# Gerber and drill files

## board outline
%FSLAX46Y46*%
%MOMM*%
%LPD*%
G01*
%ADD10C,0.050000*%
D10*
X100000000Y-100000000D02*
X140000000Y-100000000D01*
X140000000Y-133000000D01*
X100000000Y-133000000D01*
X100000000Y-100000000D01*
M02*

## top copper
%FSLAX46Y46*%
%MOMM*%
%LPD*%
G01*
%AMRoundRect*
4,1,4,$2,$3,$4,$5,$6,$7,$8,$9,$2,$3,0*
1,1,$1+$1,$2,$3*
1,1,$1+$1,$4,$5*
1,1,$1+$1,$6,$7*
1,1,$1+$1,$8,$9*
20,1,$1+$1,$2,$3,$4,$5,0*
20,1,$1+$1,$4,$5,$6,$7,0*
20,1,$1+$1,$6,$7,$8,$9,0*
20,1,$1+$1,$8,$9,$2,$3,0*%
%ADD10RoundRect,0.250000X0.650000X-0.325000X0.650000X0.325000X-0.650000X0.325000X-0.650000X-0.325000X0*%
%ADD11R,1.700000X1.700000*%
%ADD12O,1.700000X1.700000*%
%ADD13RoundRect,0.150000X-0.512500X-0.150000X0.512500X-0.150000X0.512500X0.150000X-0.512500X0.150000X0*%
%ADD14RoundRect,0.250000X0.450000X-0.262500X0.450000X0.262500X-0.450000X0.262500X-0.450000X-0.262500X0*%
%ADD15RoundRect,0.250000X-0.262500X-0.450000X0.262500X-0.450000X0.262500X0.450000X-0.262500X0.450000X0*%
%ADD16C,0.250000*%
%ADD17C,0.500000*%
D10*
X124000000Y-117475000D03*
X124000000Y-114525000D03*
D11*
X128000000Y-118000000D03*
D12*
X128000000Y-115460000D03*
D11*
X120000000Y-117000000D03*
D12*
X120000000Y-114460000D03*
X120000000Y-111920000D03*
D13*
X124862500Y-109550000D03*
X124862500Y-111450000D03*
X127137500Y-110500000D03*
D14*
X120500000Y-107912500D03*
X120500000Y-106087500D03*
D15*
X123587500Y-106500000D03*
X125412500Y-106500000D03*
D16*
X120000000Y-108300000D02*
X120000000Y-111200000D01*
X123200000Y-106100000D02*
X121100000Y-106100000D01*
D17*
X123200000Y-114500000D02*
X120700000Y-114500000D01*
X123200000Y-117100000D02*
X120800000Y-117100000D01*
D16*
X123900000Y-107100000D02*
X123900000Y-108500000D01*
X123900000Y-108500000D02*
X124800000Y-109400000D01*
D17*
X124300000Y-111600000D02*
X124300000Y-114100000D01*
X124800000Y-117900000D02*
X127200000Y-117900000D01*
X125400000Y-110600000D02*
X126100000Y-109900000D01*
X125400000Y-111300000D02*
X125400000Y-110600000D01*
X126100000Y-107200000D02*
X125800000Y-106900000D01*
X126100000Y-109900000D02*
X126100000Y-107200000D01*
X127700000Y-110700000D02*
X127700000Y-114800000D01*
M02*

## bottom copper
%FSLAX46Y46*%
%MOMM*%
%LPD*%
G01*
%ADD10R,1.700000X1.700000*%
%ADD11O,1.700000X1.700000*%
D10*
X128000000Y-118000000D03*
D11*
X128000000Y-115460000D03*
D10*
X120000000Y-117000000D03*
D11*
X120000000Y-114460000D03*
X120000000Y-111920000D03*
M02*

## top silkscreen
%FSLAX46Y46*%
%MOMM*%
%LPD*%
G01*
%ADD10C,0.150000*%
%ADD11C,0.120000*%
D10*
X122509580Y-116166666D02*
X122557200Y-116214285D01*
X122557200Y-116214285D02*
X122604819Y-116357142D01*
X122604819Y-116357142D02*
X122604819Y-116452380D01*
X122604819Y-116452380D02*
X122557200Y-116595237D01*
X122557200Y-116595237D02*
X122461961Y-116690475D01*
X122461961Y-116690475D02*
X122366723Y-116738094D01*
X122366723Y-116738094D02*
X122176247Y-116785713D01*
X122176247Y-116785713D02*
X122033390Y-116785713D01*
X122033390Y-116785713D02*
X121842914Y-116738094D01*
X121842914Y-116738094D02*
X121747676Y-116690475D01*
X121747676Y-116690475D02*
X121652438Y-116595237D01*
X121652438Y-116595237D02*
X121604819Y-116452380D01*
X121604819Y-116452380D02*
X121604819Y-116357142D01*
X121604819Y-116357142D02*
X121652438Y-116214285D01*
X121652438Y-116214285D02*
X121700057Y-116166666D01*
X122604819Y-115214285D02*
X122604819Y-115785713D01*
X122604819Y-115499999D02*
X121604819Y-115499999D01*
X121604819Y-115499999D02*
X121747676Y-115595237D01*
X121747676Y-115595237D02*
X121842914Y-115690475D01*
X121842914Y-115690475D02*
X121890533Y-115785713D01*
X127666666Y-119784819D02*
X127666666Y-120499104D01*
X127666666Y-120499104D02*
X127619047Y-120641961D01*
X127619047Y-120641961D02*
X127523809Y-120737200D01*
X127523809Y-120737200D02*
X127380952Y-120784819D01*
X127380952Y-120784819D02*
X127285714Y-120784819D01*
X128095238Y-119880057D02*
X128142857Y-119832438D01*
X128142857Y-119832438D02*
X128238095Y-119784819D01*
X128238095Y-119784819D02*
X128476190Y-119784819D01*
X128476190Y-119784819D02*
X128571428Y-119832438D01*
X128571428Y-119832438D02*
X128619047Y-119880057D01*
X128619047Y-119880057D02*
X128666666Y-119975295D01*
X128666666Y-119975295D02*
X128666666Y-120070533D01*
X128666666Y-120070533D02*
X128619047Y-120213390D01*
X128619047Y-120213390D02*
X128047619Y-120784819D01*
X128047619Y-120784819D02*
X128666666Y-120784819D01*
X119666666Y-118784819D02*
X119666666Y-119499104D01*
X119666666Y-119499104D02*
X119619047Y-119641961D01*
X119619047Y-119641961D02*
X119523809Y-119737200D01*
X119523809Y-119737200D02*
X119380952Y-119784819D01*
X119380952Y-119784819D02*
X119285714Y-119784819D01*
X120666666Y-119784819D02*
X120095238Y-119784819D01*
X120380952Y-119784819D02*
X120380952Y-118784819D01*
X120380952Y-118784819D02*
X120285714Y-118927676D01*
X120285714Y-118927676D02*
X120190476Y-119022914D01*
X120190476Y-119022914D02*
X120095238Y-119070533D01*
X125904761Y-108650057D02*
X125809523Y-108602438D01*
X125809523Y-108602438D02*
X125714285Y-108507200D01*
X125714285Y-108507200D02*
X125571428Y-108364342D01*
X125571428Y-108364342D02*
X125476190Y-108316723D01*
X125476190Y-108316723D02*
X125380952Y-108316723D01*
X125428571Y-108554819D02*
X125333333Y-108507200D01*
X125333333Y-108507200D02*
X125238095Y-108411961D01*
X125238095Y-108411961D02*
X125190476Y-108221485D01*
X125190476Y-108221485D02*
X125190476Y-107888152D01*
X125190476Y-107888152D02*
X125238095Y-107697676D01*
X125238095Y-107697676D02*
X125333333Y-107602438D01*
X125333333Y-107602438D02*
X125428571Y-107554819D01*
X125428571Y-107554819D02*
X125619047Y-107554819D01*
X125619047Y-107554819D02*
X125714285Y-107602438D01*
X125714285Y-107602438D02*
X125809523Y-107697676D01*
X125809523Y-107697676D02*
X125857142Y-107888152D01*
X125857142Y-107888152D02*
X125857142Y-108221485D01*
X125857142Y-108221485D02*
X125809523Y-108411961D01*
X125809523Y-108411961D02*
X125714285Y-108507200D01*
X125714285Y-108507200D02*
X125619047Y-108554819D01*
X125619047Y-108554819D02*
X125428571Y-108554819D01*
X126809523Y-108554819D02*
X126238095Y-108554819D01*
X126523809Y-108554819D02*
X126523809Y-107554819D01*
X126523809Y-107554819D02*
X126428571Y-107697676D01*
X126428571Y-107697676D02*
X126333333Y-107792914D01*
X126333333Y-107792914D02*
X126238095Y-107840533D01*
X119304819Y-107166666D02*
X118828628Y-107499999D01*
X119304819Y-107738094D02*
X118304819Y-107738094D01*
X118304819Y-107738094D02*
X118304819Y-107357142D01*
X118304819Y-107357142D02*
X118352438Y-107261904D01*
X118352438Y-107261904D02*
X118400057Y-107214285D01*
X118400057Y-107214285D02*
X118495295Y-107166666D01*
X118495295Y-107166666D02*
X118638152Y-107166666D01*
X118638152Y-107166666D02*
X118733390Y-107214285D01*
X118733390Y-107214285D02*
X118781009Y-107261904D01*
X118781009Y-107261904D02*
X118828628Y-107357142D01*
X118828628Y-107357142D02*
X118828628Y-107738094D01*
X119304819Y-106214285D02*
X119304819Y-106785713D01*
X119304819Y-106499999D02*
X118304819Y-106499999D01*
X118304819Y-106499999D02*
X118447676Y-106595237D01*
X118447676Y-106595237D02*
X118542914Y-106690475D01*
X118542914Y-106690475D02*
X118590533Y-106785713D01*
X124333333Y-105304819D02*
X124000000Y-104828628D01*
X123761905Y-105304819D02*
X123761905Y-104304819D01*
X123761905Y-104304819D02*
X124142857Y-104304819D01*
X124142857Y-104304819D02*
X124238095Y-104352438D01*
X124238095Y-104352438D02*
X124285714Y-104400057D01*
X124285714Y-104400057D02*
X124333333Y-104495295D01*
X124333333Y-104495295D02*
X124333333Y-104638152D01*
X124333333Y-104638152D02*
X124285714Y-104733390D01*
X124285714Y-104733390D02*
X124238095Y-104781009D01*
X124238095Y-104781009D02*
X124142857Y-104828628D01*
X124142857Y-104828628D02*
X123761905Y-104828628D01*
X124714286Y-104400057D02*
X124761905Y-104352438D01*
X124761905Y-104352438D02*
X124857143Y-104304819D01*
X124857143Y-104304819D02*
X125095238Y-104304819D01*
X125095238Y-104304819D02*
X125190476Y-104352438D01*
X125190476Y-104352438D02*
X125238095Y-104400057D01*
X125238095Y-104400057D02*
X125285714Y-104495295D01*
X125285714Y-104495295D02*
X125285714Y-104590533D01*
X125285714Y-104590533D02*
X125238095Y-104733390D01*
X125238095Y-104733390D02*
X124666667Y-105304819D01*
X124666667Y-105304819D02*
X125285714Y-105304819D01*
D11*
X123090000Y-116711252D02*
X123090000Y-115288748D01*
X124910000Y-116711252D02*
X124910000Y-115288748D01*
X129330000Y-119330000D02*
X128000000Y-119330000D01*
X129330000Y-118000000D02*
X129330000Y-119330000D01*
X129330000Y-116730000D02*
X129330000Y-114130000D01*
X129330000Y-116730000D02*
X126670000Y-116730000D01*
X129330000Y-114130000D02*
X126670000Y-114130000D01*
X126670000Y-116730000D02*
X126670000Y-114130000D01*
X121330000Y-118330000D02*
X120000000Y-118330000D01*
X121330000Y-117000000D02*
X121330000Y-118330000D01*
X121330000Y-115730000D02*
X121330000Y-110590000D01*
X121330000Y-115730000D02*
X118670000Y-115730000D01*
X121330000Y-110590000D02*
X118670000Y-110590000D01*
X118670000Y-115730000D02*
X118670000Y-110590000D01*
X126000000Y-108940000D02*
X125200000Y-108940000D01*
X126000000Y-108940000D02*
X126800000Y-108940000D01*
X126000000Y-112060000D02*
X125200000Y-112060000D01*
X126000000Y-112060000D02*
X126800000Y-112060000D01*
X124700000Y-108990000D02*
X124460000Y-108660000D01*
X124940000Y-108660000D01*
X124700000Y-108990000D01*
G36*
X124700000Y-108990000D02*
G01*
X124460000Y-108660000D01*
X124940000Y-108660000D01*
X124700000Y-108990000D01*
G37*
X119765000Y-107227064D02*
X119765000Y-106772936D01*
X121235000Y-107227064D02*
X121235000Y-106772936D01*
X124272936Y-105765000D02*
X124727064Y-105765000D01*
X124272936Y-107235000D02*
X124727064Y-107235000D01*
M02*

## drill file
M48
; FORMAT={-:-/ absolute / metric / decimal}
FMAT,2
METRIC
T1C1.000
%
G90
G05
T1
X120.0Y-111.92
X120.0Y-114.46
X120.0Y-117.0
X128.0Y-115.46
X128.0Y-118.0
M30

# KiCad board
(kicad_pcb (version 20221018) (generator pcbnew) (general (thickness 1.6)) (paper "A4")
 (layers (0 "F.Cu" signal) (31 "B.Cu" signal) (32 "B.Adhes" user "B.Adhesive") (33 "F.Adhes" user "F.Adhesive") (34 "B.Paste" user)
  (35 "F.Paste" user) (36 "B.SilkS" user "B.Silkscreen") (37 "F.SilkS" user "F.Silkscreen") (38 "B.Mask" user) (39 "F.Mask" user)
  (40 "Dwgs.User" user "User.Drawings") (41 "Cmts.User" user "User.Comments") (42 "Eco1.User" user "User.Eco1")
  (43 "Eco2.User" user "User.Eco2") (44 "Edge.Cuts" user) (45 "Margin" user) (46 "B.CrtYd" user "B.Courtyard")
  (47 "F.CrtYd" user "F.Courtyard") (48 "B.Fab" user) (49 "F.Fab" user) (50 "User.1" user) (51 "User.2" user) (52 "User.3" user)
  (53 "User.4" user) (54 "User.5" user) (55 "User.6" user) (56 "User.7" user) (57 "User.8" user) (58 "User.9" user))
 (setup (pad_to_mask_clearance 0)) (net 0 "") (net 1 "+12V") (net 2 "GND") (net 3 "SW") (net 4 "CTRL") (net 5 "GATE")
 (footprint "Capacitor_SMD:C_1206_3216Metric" (layer "F.Cu") (at 124 116 90)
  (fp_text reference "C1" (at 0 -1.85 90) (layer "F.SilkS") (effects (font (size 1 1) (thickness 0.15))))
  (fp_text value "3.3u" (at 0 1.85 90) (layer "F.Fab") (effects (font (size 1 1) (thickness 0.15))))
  (fp_line (start -0.711252 -0.91) (end 0.711252 -0.91) (stroke (width 0.12) (type solid)) (layer "F.SilkS"))
  (fp_line (start -0.711252 0.91) (end 0.711252 0.91) (stroke (width 0.12) (type solid)) (layer "F.SilkS"))
  (pad "1" smd roundrect (at -1.475 0 90) (size 1.15 1.8) (layers "F.Cu" "F.Paste" "F.Mask") (roundrect_rratio 0.217391) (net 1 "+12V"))
  (pad "2" smd roundrect (at 1.475 0 90) (size 1.15 1.8) (layers "F.Cu" "F.Paste" "F.Mask") (roundrect_rratio 0.217391) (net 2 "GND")))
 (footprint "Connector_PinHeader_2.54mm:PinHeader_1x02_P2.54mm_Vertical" (layer "F.Cu") (at 128 118 180)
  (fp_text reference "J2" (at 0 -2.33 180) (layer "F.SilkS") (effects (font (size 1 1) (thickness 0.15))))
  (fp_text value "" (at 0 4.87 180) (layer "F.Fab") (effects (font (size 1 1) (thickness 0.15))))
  (fp_line (start -1.33 -1.33) (end 0 -1.33) (stroke (width 0.12) (type solid)) (layer "F.SilkS"))
  (fp_line (start -1.33 0) (end -1.33 -1.33) (stroke (width 0.12) (type solid)) (layer "F.SilkS"))
  (fp_line (start -1.33 1.27) (end -1.33 3.87) (stroke (width 0.12) (type solid)) (layer "F.SilkS"))
  (fp_line (start -1.33 1.27) (end 1.33 1.27) (stroke (width 0.12) (type solid)) (layer "F.SilkS"))
  (fp_line (start -1.33 3.87) (end 1.33 3.87) (stroke (width 0.12) (type solid)) (layer "F.SilkS"))
  (fp_line (start 1.33 1.27) (end 1.33 3.87) (stroke (width 0.12) (type solid)) (layer "F.SilkS"))
  (pad "1" thru_hole rect (at 0 0 180) (size 1.7 1.7) (drill 1) (layers "*.Cu" "*.Mask") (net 1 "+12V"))
  (pad "2" thru_hole oval (at 0 2.54 180) (size 1.7 1.7) (drill 1) (layers "*.Cu" "*.Mask") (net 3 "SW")))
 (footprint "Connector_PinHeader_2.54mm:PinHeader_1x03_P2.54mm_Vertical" (layer "F.Cu") (at 120 117 180)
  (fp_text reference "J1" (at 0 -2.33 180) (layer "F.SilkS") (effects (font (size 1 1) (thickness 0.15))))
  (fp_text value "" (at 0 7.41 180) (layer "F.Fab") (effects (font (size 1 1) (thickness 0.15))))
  (fp_line (start -1.33 -1.33) (end 0 -1.33) (stroke (width 0.12) (type solid)) (layer "F.SilkS"))
  (fp_line (start -1.33 0) (end -1.33 -1.33) (stroke (width 0.12) (type solid)) (layer "F.SilkS"))
  (fp_line (start -1.33 1.27) (end -1.33 6.41) (stroke (width 0.12) (type solid)) (layer "F.SilkS"))
  (fp_line (start -1.33 1.27) (end 1.33 1.27) (stroke (width 0.12) (type solid)) (layer "F.SilkS"))
  (fp_line (start -1.33 6.41) (end 1.33 6.41) (stroke (width 0.12) (type solid)) (layer "F.SilkS"))
  (fp_line (start 1.33 1.27) (end 1.33 6.41) (stroke (width 0.12) (type solid)) (layer "F.SilkS"))
  (pad "1" thru_hole rect (at 0 0 180) (size 1.7 1.7) (drill 1) (layers "*.Cu" "*.Mask") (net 1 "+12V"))
  (pad "2" thru_hole oval (at 0 2.54 180) (size 1.7 1.7) (drill 1) (layers "*.Cu" "*.Mask") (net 2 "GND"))
  (pad "3" thru_hole oval (at 0 5.08 180) (size 1.7 1.7) (drill 1) (layers "*.Cu" "*.Mask") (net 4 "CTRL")))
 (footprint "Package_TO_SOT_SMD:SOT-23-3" (layer "F.Cu") (at 126 110.5)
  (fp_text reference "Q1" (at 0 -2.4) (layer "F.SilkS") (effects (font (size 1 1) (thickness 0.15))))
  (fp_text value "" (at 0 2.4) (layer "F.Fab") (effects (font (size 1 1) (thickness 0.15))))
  (fp_line (start 0 -1.56) (end -0.8 -1.56) (stroke (width 0.12) (type solid)) (layer "F.SilkS"))
  (fp_line (start 0 -1.56) (end 0.8 -1.56) (stroke (width 0.12) (type solid)) (layer "F.SilkS"))
  (fp_line (start 0 1.56) (end -0.8 1.56) (stroke (width 0.12) (type solid)) (layer "F.SilkS"))
  (fp_line (start 0 1.56) (end 0.8 1.56) (stroke (width 0.12) (type solid)) (layer "F.SilkS"))
  (fp_poly
   (pts (xy -1.3 -1.51) (xy -1.54 -1.84) (xy -1.06 -1.84) (xy -1.3 -1.51)) (stroke (width 0.12) (type solid)) (fill solid) (layer "F.SilkS"))
  (pad "1" smd roundrect (at -1.1375 -0.95) (size 1.325 0.6) (layers "F.Cu" "F.Paste" "F.Mask") (roundrect_rratio 0.25) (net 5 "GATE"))
  (pad "2" smd roundrect (at -1.1375 0.95) (size 1.325 0.6) (layers "F.Cu" "F.Paste" "F.Mask") (roundrect_rratio 0.25) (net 2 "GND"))
  (pad "3" smd roundrect (at 1.1375 0) (size 1.325 0.6) (layers "F.Cu" "F.Paste" "F.Mask") (roundrect_rratio 0.25) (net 3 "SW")))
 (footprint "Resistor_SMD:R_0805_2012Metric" (layer "F.Cu") (at 120.5 107 90)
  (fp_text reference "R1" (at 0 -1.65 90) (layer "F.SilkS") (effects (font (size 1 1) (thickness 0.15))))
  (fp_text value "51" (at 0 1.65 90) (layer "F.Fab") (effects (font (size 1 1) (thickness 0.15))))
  (fp_line (start -0.227064 -0.735) (end 0.227064 -0.735) (stroke (width 0.12) (type solid)) (layer "F.SilkS"))
  (fp_line (start -0.227064 0.735) (end 0.227064 0.735) (stroke (width 0.12) (type solid)) (layer "F.SilkS"))
  (pad "1" smd roundrect (at -0.9125 0 90) (size 1.025 1.4) (layers "F.Cu" "F.Paste" "F.Mask") (roundrect_rratio 0.243902) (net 4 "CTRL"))
  (pad "2" smd roundrect (at 0.9125 0 90) (size 1.025 1.4) (layers "F.Cu" "F.Paste" "F.Mask") (roundrect_rratio 0.243902) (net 5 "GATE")))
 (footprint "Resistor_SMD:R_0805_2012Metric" (layer "F.Cu") (at 124.5 106.5)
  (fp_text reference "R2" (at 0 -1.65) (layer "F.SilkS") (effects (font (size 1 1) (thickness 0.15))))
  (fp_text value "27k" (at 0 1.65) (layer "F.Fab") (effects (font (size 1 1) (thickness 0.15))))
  (fp_line (start -0.227064 -0.735) (end 0.227064 -0.735) (stroke (width 0.12) (type solid)) (layer "F.SilkS"))
  (fp_line (start -0.227064 0.735) (end 0.227064 0.735) (stroke (width 0.12) (type solid)) (layer "F.SilkS"))
  (pad "1" smd roundrect (at -0.9125 0) (size 1.025 1.4) (layers "F.Cu" "F.Paste" "F.Mask") (roundrect_rratio 0.243902) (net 5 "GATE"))
  (pad "2" smd roundrect (at 0.9125 0) (size 1.025 1.4) (layers "F.Cu" "F.Paste" "F.Mask") (roundrect_rratio 0.243902) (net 2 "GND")))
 (gr_rect (start 100 100) (end 140 133) (stroke (width 0.05) (type default)) (fill none) (layer "Edge.Cuts"))
 (segment (start 120 108.3) (end 120 111.2) (width 0.25) (layer "F.Cu") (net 4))
 (segment (start 123.2 106.1) (end 121.1 106.1) (width 0.25) (layer "F.Cu") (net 5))
 (segment (start 123.2 114.5) (end 120.7 114.5) (width 0.5) (layer "F.Cu") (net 2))
 (segment (start 123.2 117.1) (end 120.8 117.1) (width 0.5) (layer "F.Cu") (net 1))
 (segment (start 123.9 107.1) (end 123.9 108.5) (width 0.25) (layer "F.Cu") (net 5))
 (segment (start 123.9 108.5) (end 124.8 109.4) (width 0.25) (layer "F.Cu") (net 5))
 (segment (start 124.3 111.6) (end 124.3 114.1) (width 0.5) (layer "F.Cu") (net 2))
 (segment (start 124.8 117.9) (end 127.2 117.9) (width 0.5) (layer "F.Cu") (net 1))
 (segment (start 125.4 110.6) (end 126.1 109.9) (width 0.5) (layer "F.Cu") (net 2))
 (segment (start 125.4 111.3) (end 125.4 110.6) (width 0.5) (layer "F.Cu") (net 2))
 (segment (start 126.1 107.2) (end 125.8 106.9) (width 0.5) (layer "F.Cu") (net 2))
 (segment (start 126.1 109.9) (end 126.1 107.2) (width 0.5) (layer "F.Cu") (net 2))
 (segment (start 127.7 110.7) (end 127.7 114.8) (width 0.5) (layer "F.Cu") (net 3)))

